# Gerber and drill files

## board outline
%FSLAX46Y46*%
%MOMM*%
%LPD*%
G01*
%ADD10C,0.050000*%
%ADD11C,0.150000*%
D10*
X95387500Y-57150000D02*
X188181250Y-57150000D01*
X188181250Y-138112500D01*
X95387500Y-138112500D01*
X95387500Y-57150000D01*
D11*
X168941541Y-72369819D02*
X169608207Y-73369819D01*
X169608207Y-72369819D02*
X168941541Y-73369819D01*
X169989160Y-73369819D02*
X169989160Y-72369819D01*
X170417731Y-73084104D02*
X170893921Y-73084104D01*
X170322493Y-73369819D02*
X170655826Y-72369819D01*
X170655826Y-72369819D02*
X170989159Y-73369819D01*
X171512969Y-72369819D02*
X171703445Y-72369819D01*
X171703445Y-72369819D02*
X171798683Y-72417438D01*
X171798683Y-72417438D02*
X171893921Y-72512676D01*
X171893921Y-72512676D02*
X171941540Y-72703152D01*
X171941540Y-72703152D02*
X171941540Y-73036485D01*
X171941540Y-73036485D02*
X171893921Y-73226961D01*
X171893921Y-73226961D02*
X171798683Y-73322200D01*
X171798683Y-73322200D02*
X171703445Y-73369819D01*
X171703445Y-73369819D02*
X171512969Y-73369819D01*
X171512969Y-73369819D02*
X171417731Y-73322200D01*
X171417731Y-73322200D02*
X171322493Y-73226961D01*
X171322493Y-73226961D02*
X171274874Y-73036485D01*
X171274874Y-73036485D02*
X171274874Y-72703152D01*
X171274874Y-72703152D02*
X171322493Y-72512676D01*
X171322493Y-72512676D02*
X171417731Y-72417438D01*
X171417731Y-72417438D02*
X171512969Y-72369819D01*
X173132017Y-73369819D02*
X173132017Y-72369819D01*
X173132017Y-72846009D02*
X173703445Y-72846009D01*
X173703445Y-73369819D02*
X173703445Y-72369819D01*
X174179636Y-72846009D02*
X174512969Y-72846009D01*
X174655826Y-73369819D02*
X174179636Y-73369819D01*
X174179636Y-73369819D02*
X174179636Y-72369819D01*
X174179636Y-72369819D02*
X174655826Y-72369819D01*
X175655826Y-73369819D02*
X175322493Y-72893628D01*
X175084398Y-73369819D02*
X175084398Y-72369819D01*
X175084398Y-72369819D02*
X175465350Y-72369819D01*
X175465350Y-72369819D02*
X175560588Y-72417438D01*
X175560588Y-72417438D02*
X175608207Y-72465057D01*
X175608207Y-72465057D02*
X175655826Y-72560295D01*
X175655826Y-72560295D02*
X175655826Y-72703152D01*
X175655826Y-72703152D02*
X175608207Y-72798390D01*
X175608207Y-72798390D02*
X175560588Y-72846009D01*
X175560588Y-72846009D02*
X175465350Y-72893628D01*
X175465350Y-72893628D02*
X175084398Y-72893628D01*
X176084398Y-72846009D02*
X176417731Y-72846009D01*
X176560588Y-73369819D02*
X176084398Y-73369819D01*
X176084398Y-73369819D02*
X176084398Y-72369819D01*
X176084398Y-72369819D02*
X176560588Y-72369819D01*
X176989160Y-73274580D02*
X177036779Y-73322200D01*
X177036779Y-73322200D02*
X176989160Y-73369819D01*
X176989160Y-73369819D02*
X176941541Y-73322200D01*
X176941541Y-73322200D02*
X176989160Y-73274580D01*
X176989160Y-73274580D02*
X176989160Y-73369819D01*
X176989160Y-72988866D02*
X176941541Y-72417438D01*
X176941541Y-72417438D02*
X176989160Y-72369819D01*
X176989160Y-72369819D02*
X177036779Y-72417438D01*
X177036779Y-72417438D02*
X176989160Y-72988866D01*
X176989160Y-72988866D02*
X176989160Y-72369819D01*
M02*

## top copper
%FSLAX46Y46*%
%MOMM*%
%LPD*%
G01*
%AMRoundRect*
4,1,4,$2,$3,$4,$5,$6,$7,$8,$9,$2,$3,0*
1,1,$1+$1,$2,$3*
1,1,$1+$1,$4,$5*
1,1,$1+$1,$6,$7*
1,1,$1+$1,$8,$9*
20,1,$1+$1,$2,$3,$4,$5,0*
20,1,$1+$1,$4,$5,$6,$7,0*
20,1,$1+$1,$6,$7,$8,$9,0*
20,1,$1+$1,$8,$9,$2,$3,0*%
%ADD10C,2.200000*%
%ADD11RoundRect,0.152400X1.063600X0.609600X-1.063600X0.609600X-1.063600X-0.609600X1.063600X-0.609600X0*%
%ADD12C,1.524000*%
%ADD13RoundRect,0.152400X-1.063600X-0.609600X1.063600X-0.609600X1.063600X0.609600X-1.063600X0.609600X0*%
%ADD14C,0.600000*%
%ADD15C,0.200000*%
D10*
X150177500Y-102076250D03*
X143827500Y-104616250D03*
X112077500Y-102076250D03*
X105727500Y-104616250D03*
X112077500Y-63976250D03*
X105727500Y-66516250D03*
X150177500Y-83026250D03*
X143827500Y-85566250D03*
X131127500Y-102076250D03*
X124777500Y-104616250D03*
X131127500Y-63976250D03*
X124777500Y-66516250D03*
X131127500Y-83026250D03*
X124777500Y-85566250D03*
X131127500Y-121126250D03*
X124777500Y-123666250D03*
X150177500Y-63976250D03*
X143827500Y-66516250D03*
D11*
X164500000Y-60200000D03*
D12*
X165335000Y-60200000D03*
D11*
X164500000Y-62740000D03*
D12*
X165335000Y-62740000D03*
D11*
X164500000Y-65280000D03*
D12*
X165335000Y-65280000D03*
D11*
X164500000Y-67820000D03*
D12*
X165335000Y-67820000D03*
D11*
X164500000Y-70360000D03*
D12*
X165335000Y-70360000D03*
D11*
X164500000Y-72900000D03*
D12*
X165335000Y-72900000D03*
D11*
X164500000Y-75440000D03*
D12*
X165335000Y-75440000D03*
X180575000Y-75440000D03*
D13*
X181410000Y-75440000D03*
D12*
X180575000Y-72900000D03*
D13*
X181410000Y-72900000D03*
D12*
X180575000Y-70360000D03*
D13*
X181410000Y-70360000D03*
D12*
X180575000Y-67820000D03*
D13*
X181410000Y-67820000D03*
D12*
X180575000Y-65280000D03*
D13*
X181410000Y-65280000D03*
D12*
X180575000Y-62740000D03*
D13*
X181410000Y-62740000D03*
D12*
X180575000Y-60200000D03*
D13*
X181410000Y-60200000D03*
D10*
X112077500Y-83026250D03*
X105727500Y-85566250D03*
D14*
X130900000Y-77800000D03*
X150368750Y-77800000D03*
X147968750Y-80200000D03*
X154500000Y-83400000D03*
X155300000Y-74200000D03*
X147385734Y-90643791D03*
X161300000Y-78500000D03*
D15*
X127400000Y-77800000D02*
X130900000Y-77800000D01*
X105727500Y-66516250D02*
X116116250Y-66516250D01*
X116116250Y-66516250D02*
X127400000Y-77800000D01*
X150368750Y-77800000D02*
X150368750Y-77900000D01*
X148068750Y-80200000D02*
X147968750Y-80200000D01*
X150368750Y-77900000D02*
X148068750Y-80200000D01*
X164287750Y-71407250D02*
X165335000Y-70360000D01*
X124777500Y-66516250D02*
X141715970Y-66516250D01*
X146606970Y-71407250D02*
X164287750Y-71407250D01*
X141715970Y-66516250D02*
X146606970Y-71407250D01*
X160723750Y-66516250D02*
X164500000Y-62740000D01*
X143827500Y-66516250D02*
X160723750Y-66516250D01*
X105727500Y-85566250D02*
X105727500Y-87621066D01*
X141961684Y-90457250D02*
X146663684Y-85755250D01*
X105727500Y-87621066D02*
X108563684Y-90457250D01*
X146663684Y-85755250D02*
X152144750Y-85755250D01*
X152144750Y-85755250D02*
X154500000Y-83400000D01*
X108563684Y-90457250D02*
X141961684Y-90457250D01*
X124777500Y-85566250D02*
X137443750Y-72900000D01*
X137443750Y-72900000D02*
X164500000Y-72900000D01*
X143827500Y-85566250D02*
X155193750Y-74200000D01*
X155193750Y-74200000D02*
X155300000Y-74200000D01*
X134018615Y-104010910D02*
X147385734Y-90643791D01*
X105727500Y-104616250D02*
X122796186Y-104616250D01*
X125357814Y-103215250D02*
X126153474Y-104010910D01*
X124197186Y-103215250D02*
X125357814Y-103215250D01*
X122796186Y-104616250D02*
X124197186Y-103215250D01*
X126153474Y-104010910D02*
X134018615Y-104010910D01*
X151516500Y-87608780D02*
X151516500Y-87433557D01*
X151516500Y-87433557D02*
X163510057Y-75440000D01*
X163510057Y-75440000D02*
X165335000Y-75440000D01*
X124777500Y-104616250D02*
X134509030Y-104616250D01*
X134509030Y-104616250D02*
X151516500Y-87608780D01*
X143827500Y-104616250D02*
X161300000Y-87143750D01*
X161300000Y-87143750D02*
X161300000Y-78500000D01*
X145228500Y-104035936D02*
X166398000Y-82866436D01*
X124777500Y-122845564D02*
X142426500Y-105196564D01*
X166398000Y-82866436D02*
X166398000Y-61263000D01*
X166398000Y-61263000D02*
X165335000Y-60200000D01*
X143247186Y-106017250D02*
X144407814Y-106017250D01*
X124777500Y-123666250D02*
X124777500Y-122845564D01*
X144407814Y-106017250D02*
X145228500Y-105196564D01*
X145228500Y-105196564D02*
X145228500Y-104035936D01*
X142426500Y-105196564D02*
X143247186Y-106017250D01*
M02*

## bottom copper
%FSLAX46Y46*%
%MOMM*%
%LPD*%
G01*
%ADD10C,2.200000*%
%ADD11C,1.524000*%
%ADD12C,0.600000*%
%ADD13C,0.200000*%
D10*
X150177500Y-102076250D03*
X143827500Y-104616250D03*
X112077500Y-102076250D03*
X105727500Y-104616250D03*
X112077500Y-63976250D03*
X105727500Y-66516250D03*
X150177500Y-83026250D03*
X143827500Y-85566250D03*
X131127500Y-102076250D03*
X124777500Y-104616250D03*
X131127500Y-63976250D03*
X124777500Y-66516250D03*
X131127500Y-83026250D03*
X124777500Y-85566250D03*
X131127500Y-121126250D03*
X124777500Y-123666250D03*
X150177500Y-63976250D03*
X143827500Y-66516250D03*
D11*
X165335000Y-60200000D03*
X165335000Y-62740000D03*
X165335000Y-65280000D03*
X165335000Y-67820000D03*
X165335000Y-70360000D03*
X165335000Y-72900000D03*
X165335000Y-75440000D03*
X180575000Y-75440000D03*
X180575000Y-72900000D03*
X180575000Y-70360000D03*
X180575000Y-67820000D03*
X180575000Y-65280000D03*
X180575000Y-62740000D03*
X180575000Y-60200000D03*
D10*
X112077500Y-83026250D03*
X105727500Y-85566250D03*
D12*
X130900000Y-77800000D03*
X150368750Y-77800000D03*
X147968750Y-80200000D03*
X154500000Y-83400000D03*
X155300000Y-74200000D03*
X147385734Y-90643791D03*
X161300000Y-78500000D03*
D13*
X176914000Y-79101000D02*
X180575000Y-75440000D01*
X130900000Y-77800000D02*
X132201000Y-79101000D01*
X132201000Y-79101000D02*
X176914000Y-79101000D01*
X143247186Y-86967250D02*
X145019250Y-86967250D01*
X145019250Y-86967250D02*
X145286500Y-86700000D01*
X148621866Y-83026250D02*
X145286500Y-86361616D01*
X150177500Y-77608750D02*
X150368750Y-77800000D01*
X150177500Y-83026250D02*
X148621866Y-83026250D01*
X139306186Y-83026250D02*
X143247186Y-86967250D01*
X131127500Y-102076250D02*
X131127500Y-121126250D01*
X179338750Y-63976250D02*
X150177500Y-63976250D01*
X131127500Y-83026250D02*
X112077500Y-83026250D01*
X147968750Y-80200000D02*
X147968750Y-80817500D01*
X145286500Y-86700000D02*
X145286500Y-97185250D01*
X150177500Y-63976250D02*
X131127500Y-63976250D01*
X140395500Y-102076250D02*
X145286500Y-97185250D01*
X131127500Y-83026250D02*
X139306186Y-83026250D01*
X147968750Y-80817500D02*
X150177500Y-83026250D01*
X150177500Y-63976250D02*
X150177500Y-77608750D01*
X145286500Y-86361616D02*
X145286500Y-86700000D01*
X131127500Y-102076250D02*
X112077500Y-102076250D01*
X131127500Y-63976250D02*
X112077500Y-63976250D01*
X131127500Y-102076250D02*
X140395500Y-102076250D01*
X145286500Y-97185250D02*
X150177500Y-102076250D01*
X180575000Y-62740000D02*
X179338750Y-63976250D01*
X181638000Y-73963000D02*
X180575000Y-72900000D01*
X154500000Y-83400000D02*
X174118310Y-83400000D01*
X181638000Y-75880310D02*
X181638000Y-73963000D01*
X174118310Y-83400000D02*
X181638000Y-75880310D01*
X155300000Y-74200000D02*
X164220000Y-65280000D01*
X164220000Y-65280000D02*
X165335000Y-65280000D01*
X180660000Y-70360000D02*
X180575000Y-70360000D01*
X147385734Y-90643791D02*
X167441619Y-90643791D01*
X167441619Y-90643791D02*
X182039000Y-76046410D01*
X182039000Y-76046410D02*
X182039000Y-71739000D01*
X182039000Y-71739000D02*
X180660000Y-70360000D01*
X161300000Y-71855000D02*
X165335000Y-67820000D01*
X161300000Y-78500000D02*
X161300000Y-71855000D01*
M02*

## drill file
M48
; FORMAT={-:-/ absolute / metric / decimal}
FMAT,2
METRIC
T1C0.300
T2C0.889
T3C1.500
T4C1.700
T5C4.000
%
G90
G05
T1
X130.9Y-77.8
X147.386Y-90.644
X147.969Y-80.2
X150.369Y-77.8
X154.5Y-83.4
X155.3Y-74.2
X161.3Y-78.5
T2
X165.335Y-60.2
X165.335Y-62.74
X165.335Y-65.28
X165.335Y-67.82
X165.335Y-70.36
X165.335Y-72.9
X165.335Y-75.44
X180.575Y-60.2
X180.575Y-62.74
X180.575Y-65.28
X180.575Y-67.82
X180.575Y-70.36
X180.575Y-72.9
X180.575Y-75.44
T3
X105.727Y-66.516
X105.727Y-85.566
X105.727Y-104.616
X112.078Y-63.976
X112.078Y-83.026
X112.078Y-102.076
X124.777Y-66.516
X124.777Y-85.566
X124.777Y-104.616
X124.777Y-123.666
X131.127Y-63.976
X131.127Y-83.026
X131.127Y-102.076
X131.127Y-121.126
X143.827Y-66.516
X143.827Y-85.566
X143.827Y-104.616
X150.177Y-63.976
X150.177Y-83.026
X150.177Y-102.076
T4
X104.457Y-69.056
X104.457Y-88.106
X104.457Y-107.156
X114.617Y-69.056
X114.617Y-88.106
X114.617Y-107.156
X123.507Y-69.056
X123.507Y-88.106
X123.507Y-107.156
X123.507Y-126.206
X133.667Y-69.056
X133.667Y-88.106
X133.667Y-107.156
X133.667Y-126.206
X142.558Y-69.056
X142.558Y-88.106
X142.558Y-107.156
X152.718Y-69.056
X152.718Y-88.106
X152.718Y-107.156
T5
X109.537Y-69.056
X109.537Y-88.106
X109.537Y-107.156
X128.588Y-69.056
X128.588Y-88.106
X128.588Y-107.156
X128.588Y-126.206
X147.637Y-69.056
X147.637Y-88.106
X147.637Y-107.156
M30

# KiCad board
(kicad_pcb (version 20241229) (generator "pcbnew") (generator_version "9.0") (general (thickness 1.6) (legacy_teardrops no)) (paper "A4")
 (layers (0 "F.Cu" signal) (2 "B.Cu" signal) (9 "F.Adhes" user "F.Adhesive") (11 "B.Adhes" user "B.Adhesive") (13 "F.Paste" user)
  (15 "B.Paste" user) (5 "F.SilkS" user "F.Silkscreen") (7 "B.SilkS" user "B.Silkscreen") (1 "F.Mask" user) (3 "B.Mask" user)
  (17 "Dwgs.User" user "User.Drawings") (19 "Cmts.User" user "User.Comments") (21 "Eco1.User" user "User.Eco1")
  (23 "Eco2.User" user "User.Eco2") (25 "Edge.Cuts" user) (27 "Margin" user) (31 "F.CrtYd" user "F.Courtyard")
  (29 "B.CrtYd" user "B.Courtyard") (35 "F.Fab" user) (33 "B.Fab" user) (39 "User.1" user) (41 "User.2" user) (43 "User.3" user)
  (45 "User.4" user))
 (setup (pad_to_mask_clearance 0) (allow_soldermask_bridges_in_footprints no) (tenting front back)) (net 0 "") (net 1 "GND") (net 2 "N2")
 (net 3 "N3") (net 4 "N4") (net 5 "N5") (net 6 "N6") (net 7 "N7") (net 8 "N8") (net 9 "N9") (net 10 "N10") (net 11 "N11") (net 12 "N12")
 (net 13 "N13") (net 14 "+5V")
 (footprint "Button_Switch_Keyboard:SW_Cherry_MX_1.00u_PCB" (layer "F.Cu") (at 150.1775 102.07625)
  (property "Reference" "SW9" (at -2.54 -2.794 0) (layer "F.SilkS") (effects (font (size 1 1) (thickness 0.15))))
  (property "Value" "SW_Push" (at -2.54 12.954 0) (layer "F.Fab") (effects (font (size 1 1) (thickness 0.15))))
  (pad "" np_thru_hole circle (at -7.62 5.08) (size 1.7 1.7) (drill 1.7) (layers "*.Cu" "*.Mask"))
  (pad "" np_thru_hole circle (at -2.54 5.08) (size 4 4) (drill 4) (layers "*.Cu" "*.Mask"))
  (pad "" np_thru_hole circle (at 2.54 5.08) (size 1.7 1.7) (drill 1.7) (layers "*.Cu" "*.Mask"))
  (pad "1" thru_hole circle (at 0 0) (size 2.2 2.2) (drill 1.5) (layers "*.Cu" "*.Mask") (remove_unused_layers no) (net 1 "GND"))
  (pad "2" thru_hole circle (at -6.35 2.54) (size 2.2 2.2) (drill 1.5) (layers "*.Cu" "*.Mask") (remove_unused_layers no) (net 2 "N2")))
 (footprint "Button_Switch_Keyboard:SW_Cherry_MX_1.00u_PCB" (layer "F.Cu") (at 112.0775 102.07625)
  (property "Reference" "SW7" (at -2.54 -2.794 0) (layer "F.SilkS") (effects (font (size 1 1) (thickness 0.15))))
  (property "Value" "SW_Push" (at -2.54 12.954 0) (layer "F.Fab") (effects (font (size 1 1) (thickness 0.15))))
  (pad "" np_thru_hole circle (at -7.62 5.08) (size 1.7 1.7) (drill 1.7) (layers "*.Cu" "*.Mask"))
  (pad "" np_thru_hole circle (at -2.54 5.08) (size 4 4) (drill 4) (layers "*.Cu" "*.Mask"))
  (pad "" np_thru_hole circle (at 2.54 5.08) (size 1.7 1.7) (drill 1.7) (layers "*.Cu" "*.Mask"))
  (pad "1" thru_hole circle (at 0 0) (size 2.2 2.2) (drill 1.5) (layers "*.Cu" "*.Mask") (remove_unused_layers no) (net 1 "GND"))
  (pad "2" thru_hole circle (at -6.35 2.54) (size 2.2 2.2) (drill 1.5) (layers "*.Cu" "*.Mask") (remove_unused_layers no) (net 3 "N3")))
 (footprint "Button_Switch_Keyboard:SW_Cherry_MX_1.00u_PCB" (layer "F.Cu") (at 112.0775 63.97625)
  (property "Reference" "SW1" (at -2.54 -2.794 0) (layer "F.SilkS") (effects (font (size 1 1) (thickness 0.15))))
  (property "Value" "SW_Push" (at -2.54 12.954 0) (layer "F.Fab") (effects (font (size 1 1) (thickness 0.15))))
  (pad "" np_thru_hole circle (at -7.62 5.08) (size 1.7 1.7) (drill 1.7) (layers "*.Cu" "*.Mask"))
  (pad "" np_thru_hole circle (at -2.54 5.08) (size 4 4) (drill 4) (layers "*.Cu" "*.Mask"))
  (pad "" np_thru_hole circle (at 2.54 5.08) (size 1.7 1.7) (drill 1.7) (layers "*.Cu" "*.Mask"))
  (pad "1" thru_hole circle (at 0 0) (size 2.2 2.2) (drill 1.5) (layers "*.Cu" "*.Mask") (remove_unused_layers no) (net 1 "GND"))
  (pad "2" thru_hole circle (at -6.35 2.54) (size 2.2 2.2) (drill 1.5) (layers "*.Cu" "*.Mask") (remove_unused_layers no) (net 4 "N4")))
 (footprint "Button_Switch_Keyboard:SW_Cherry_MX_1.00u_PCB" (layer "F.Cu") (at 150.1775 83.02625)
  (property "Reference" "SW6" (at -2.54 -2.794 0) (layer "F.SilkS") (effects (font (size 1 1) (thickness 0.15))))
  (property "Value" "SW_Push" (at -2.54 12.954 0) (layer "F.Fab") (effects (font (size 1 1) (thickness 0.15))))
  (pad "" np_thru_hole circle (at -7.62 5.08) (size 1.7 1.7) (drill 1.7) (layers "*.Cu" "*.Mask"))
  (pad "" np_thru_hole circle (at -2.54 5.08) (size 4 4) (drill 4) (layers "*.Cu" "*.Mask"))
  (pad "" np_thru_hole circle (at 2.54 5.08) (size 1.7 1.7) (drill 1.7) (layers "*.Cu" "*.Mask"))
  (pad "1" thru_hole circle (at 0 0) (size 2.2 2.2) (drill 1.5) (layers "*.Cu" "*.Mask") (remove_unused_layers no) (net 1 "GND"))
  (pad "2" thru_hole circle (at -6.35 2.54) (size 2.2 2.2) (drill 1.5) (layers "*.Cu" "*.Mask") (remove_unused_layers no) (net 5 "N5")))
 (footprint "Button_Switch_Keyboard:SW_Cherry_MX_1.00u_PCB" (layer "F.Cu") (at 131.1275 102.07625)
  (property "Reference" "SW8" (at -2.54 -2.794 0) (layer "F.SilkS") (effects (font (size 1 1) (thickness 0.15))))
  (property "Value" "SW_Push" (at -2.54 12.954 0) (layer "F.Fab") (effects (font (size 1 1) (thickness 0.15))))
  (pad "" np_thru_hole circle (at -7.62 5.08) (size 1.7 1.7) (drill 1.7) (layers "*.Cu" "*.Mask"))
  (pad "" np_thru_hole circle (at -2.54 5.08) (size 4 4) (drill 4) (layers "*.Cu" "*.Mask"))
  (pad "" np_thru_hole circle (at 2.54 5.08) (size 1.7 1.7) (drill 1.7) (layers "*.Cu" "*.Mask"))
  (pad "1" thru_hole circle (at 0 0) (size 2.2 2.2) (drill 1.5) (layers "*.Cu" "*.Mask") (remove_unused_layers no) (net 1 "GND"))
  (pad "2" thru_hole circle (at -6.35 2.54) (size 2.2 2.2) (drill 1.5) (layers "*.Cu" "*.Mask") (remove_unused_layers no) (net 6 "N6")))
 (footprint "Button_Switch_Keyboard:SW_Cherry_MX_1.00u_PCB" (layer "F.Cu") (at 131.1275 63.97625)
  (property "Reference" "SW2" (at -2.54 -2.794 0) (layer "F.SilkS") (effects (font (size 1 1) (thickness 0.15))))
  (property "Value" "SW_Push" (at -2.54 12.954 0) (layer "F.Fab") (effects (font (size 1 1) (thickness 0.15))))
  (pad "" np_thru_hole circle (at -7.62 5.08) (size 1.7 1.7) (drill 1.7) (layers "*.Cu" "*.Mask"))
  (pad "" np_thru_hole circle (at -2.54 5.08) (size 4 4) (drill 4) (layers "*.Cu" "*.Mask"))
  (pad "" np_thru_hole circle (at 2.54 5.08) (size 1.7 1.7) (drill 1.7) (layers "*.Cu" "*.Mask"))
  (pad "1" thru_hole circle (at 0 0) (size 2.2 2.2) (drill 1.5) (layers "*.Cu" "*.Mask") (remove_unused_layers no) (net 1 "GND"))
  (pad "2" thru_hole circle (at -6.35 2.54) (size 2.2 2.2) (drill 1.5) (layers "*.Cu" "*.Mask") (remove_unused_layers no) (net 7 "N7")))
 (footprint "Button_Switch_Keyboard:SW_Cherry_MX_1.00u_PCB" (layer "F.Cu") (at 131.1275 83.02625)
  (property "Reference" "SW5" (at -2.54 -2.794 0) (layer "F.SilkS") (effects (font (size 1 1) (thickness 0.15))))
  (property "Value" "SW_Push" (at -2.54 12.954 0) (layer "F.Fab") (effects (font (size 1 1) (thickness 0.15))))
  (pad "" np_thru_hole circle (at -7.62 5.08) (size 1.7 1.7) (drill 1.7) (layers "*.Cu" "*.Mask"))
  (pad "" np_thru_hole circle (at -2.54 5.08) (size 4 4) (drill 4) (layers "*.Cu" "*.Mask"))
  (pad "" np_thru_hole circle (at 2.54 5.08) (size 1.7 1.7) (drill 1.7) (layers "*.Cu" "*.Mask"))
  (pad "1" thru_hole circle (at 0 0) (size 2.2 2.2) (drill 1.5) (layers "*.Cu" "*.Mask") (remove_unused_layers no) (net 1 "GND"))
  (pad "2" thru_hole circle (at -6.35 2.54) (size 2.2 2.2) (drill 1.5) (layers "*.Cu" "*.Mask") (remove_unused_layers no) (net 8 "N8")))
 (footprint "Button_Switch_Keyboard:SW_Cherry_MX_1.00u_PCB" (layer "F.Cu") (at 131.1275 121.12625)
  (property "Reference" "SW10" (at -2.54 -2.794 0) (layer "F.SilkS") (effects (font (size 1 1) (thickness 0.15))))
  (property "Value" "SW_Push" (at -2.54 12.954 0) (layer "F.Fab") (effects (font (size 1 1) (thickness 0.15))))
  (pad "" np_thru_hole circle (at -7.62 5.08) (size 1.7 1.7) (drill 1.7) (layers "*.Cu" "*.Mask"))
  (pad "" np_thru_hole circle (at -2.54 5.08) (size 4 4) (drill 4) (layers "*.Cu" "*.Mask"))
  (pad "" np_thru_hole circle (at 2.54 5.08) (size 1.7 1.7) (drill 1.7) (layers "*.Cu" "*.Mask"))
  (pad "1" thru_hole circle (at 0 0) (size 2.2 2.2) (drill 1.5) (layers "*.Cu" "*.Mask") (remove_unused_layers no) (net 1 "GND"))
  (pad "2" thru_hole circle (at -6.35 2.54) (size 2.2 2.2) (drill 1.5) (layers "*.Cu" "*.Mask") (remove_unused_layers no) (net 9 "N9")))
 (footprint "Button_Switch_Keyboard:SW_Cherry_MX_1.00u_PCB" (layer "F.Cu") (at 150.1775 63.97625)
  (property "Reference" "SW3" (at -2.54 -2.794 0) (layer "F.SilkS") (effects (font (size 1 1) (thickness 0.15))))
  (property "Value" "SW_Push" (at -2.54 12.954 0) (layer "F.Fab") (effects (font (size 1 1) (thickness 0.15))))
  (pad "" np_thru_hole circle (at -7.62 5.08) (size 1.7 1.7) (drill 1.7) (layers "*.Cu" "*.Mask"))
  (pad "" np_thru_hole circle (at -2.54 5.08) (size 4 4) (drill 4) (layers "*.Cu" "*.Mask"))
  (pad "" np_thru_hole circle (at 2.54 5.08) (size 1.7 1.7) (drill 1.7) (layers "*.Cu" "*.Mask"))
  (pad "1" thru_hole circle (at 0 0) (size 2.2 2.2) (drill 1.5) (layers "*.Cu" "*.Mask") (remove_unused_layers no) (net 1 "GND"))
  (pad "2" thru_hole circle (at -6.35 2.54) (size 2.2 2.2) (drill 1.5) (layers "*.Cu" "*.Mask") (remove_unused_layers no) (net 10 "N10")))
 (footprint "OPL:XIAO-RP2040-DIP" (layer "F.Cu") (at 172.955 67.82)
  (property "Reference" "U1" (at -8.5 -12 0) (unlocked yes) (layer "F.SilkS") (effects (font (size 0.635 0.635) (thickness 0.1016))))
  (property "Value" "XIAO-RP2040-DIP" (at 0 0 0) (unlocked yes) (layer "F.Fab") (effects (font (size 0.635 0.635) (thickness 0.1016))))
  (pad "1" smd roundrect (at -8.455 -7.62 180) (size 2.432 1.524) (layers "F.Cu" "F.Mask") (roundrect_rratio 0.1) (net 9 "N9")
   (thermal_bridge_angle 45))
  (pad "1" thru_hole circle (at -7.62 -7.62 180) (size 1.524 1.524) (drill 0.889) (layers "*.Cu" "*.Mask") (remove_unused_layers no)
   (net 9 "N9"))
  (pad "2" smd roundrect (at -8.455 -5.08 180) (size 2.432 1.524) (layers "F.Cu" "F.Mask") (roundrect_rratio 0.1) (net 10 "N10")
   (thermal_bridge_angle 45))
  (pad "2" thru_hole circle (at -7.62 -5.08 180) (size 1.524 1.524) (drill 0.889) (layers "*.Cu" "*.Mask") (remove_unused_layers no)
   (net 10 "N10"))
  (pad "3" smd roundrect (at -8.455 -2.54 180) (size 2.432 1.524) (layers "F.Cu" "F.Mask") (roundrect_rratio 0.1) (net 5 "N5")
   (thermal_bridge_angle 45))
  (pad "3" thru_hole circle (at -7.62 -2.54 180) (size 1.524 1.524) (drill 0.889) (layers "*.Cu" "*.Mask") (remove_unused_layers no)
   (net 5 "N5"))
  (pad "4" smd roundrect (at -8.455 0 180) (size 2.432 1.524) (layers "F.Cu" "F.Mask") (roundrect_rratio 0.1) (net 2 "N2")
   (thermal_bridge_angle 45))
  (pad "4" thru_hole circle (at -7.62 0 180) (size 1.524 1.524) (drill 0.889) (layers "*.Cu" "*.Mask") (remove_unused_layers no)
   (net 2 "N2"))
  (pad "5" smd roundrect (at -8.455 2.54 180) (size 2.432 1.524) (layers "F.Cu" "F.Mask") (roundrect_rratio 0.1) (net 7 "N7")
   (thermal_bridge_angle 45))
  (pad "5" thru_hole circle (at -7.62 2.54 180) (size 1.524 1.524) (drill 0.889) (layers "*.Cu" "*.Mask") (remove_unused_layers no)
   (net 7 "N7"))
  (pad "6" smd roundrect (at -8.455 5.08 180) (size 2.432 1.524) (layers "F.Cu" "F.Mask") (roundrect_rratio 0.1) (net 8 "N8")
   (thermal_bridge_angle 45))
  (pad "6" thru_hole circle (at -7.62 5.08 180) (size 1.524 1.524) (drill 0.889) (layers "*.Cu" "*.Mask") (remove_unused_layers no)
   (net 8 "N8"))
  (pad "7" smd roundrect (at -8.455 7.62 180) (size 2.432 1.524) (layers "F.Cu" "F.Mask") (roundrect_rratio 0.1) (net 6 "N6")
   (thermal_bridge_angle 45))
  (pad "7" thru_hole circle (at -7.62 7.62 180) (size 1.524 1.524) (drill 0.889) (layers "*.Cu" "*.Mask") (remove_unused_layers no)
   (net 6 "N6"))
  (pad "8" thru_hole circle (at 7.62 7.62) (size 1.524 1.524) (drill 0.889) (layers "*.Cu" "*.Mask") (remove_unused_layers no) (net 4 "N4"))
  (pad "8" smd roundrect (at 8.455 7.62) (size 2.432 1.524) (layers "F.Cu" "F.Mask") (roundrect_rratio 0.1) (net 4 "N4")
   (thermal_bridge_angle 45))
  (pad "9" thru_hole circle (at 7.62 5.08) (size 1.524 1.524) (drill 0.889) (layers "*.Cu" "*.Mask") (remove_unused_layers no)
   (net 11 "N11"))
  (pad "9" smd roundrect (at 8.455 5.08) (size 2.432 1.524) (layers "F.Cu" "F.Mask") (roundrect_rratio 0.1) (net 11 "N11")
   (thermal_bridge_angle 45))
  (pad "10" thru_hole circle (at 7.62 2.54) (size 1.524 1.524) (drill 0.889) (layers "*.Cu" "*.Mask") (remove_unused_layers no) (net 3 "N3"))
  (pad "10" smd roundrect (at 8.455 2.54) (size 2.432 1.524) (layers "F.Cu" "F.Mask") (roundrect_rratio 0.1) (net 3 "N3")
   (thermal_bridge_angle 45))
  (pad "11" thru_hole circle (at 7.62 0) (size 1.524 1.524) (drill 0.889) (layers "*.Cu" "*.Mask") (remove_unused_layers no) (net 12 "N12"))
  (pad "11" smd roundrect (at 8.455 0) (size 2.432 1.524) (layers "F.Cu" "F.Mask") (roundrect_rratio 0.1) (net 12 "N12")
   (thermal_bridge_angle 45))
  (pad "12" thru_hole circle (at 7.62 -2.54) (size 1.524 1.524) (drill 0.889) (layers "*.Cu" "*.Mask") (remove_unused_layers no)
   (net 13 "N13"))
  (pad "12" smd roundrect (at 8.455 -2.54) (size 2.432 1.524) (layers "F.Cu" "F.Mask") (roundrect_rratio 0.1) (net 13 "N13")
   (thermal_bridge_angle 45))
  (pad "13" thru_hole circle (at 7.62 -5.08) (size 1.524 1.524) (drill 0.889) (layers "*.Cu" "*.Mask") (remove_unused_layers no)
   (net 1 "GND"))
  (pad "13" smd roundrect (at 8.455 -5.08) (size 2.432 1.524) (layers "F.Cu" "F.Mask") (roundrect_rratio 0.1) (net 1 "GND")
   (thermal_bridge_angle 45))
  (pad "14" thru_hole circle (at 7.62 -7.62) (size 1.524 1.524) (drill 0.889) (layers "*.Cu" "*.Mask") (remove_unused_layers no)
   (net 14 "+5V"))
  (pad "14" smd roundrect (at 8.455 -7.62) (size 2.432 1.524) (layers "F.Cu" "F.Mask") (roundrect_rratio 0.1) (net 14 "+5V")
   (thermal_bridge_angle 45)))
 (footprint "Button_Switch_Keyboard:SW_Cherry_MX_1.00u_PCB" (layer "F.Cu") (at 112.0775 83.02625)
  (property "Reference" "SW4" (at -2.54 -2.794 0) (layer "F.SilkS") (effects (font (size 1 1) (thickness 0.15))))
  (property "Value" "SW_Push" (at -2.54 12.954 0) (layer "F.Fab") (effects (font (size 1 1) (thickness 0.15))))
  (pad "" np_thru_hole circle (at -7.62 5.08) (size 1.7 1.7) (drill 1.7) (layers "*.Cu" "*.Mask"))
  (pad "" np_thru_hole circle (at -2.54 5.08) (size 4 4) (drill 4) (layers "*.Cu" "*.Mask"))
  (pad "" np_thru_hole circle (at 2.54 5.08) (size 1.7 1.7) (drill 1.7) (layers "*.Cu" "*.Mask"))
  (pad "1" thru_hole circle (at 0 0) (size 2.2 2.2) (drill 1.5) (layers "*.Cu" "*.Mask") (remove_unused_layers no) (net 1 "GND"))
  (pad "2" thru_hole circle (at -6.35 2.54) (size 2.2 2.2) (drill 1.5) (layers "*.Cu" "*.Mask") (remove_unused_layers no) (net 11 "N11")))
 (gr_rect (start 95.3875 57.15) (end 188.18125 138.1125) (stroke (width 0.05) (type solid)) (fill no) (layer "Edge.Cuts"))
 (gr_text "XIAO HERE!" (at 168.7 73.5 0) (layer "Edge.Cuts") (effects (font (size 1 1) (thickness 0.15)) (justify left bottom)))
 (segment (start 127.4 77.8) (end 130.9 77.8) (width 0.2) (layer "F.Cu") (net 4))
 (segment (start 105.7275 66.51625) (end 116.11625 66.51625) (width 0.2) (layer "F.Cu") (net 4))
 (segment (start 116.11625 66.51625) (end 127.4 77.8) (width 0.2) (layer "F.Cu") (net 4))
 (via (at 130.9 77.8) (size 0.6) (drill 0.3) (layers "F.Cu" "B.Cu") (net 4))
 (segment (start 176.914 79.101) (end 180.575 75.44) (width 0.2) (layer "B.Cu") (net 4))
 (segment (start 130.9 77.8) (end 132.201 79.101) (width 0.2) (layer "B.Cu") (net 4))
 (segment (start 132.201 79.101) (end 176.914 79.101) (width 0.2) (layer "B.Cu") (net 4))
 (segment (start 150.36875 77.8) (end 150.36875 77.9) (width 0.2) (layer "F.Cu") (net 1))
 (segment (start 148.06875 80.2) (end 147.96875 80.2) (width 0.2) (layer "F.Cu") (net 1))
 (segment (start 150.36875 77.9) (end 148.06875 80.2) (width 0.2) (layer "F.Cu") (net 1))
 (via (at 150.36875 77.8) (size 0.6) (drill 0.3) (layers "F.Cu" "B.Cu") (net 1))
 (via (at 147.96875 80.2) (size 0.6) (drill 0.3) (layers "F.Cu" "B.Cu") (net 1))
 (segment (start 143.247186 86.96725) (end 145.01925 86.96725) (width 0.2) (layer "B.Cu") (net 1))
 (segment (start 145.01925 86.96725) (end 145.2865 86.7) (width 0.2) (layer "B.Cu") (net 1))
 (segment (start 148.621866 83.02625) (end 145.2865 86.361616) (width 0.2) (layer "B.Cu") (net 1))
 (segment (start 150.1775 77.60875) (end 150.36875 77.8) (width 0.2) (layer "B.Cu") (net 1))
 (segment (start 150.1775 83.02625) (end 148.621866 83.02625) (width 0.2) (layer "B.Cu") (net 1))
 (segment (start 139.306186 83.02625) (end 143.247186 86.96725) (width 0.2) (layer "B.Cu") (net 1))
 (segment (start 131.1275 102.07625) (end 131.1275 121.12625) (width 0.2) (layer "B.Cu") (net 1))
 (segment (start 179.33875 63.97625) (end 150.1775 63.97625) (width 0.2) (layer "B.Cu") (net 1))
 (segment (start 131.1275 83.02625) (end 112.0775 83.02625) (width 0.2) (layer "B.Cu") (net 1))
 (segment (start 147.96875 80.2) (end 147.96875 80.8175) (width 0.2) (layer "B.Cu") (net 1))
 (segment (start 145.2865 86.7) (end 145.2865 97.18525) (width 0.2) (layer "B.Cu") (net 1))
 (segment (start 150.1775 63.97625) (end 131.1275 63.97625) (width 0.2) (layer "B.Cu") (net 1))
 (segment (start 140.3955 102.07625) (end 145.2865 97.18525) (width 0.2) (layer "B.Cu") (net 1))
 (segment (start 131.1275 83.02625) (end 139.306186 83.02625) (width 0.2) (layer "B.Cu") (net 1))
 (segment (start 147.96875 80.8175) (end 150.1775 83.02625) (width 0.2) (layer "B.Cu") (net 1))
 (segment (start 150.1775 63.97625) (end 150.1775 77.60875) (width 0.2) (layer "B.Cu") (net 1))
 (segment (start 145.2865 86.361616) (end 145.2865 86.7) (width 0.2) (layer "B.Cu") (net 1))
 (segment (start 131.1275 102.07625) (end 112.0775 102.07625) (width 0.2) (layer "B.Cu") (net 1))
 (segment (start 131.1275 63.97625) (end 112.0775 63.97625) (width 0.2) (layer "B.Cu") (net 1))
 (segment (start 131.1275 102.07625) (end 140.3955 102.07625) (width 0.2) (layer "B.Cu") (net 1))
 (segment (start 145.2865 97.18525) (end 150.1775 102.07625) (width 0.2) (layer "B.Cu") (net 1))
 (segment (start 180.575 62.74) (end 179.33875 63.97625) (width 0.2) (layer "B.Cu") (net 1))
 (segment (start 164.28775 71.40725) (end 165.335 70.36) (width 0.2) (layer "F.Cu") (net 7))
 (segment (start 124.7775 66.51625) (end 141.71597 66.51625) (width 0.2) (layer "F.Cu") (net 7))
 (segment (start 146.60697 71.40725) (end 164.28775 71.40725) (width 0.2) (layer "F.Cu") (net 7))
 (segment (start 141.71597 66.51625) (end 146.60697 71.40725) (width 0.2) (layer "F.Cu") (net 7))
 (segment (start 160.72375 66.51625) (end 164.5 62.74) (width 0.2) (layer "F.Cu") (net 10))
 (segment (start 143.8275 66.51625) (end 160.72375 66.51625) (width 0.2) (layer "F.Cu") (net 10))
 (segment (start 105.7275 85.56625) (end 105.7275 87.621066) (width 0.2) (layer "F.Cu") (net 11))
 (segment (start 141.961684 90.45725) (end 146.663684 85.75525) (width 0.2) (layer "F.Cu") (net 11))
 (segment (start 105.7275 87.621066) (end 108.563684 90.45725) (width 0.2) (layer "F.Cu") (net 11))
 (segment (start 146.663684 85.75525) (end 152.14475 85.75525) (width 0.2) (layer "F.Cu") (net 11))
 (segment (start 152.14475 85.75525) (end 154.5 83.4) (width 0.2) (layer "F.Cu") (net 11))
 (segment (start 108.563684 90.45725) (end 141.961684 90.45725) (width 0.2) (layer "F.Cu") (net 11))
 (via (at 154.5 83.4) (size 0.6) (drill 0.3) (layers "F.Cu" "B.Cu") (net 11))
 (segment (start 181.638 73.963) (end 180.575 72.9) (width 0.2) (layer "B.Cu") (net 11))
 (segment (start 154.5 83.4) (end 174.11831 83.4) (width 0.2) (layer "B.Cu") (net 11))
 (segment (start 181.638 75.88031) (end 181.638 73.963) (width 0.2) (layer "B.Cu") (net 11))
 (segment (start 174.11831 83.4) (end 181.638 75.88031) (width 0.2) (layer "B.Cu") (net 11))
 (segment (start 124.7775 85.56625) (end 137.44375 72.9) (width 0.2) (layer "F.Cu") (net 8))
 (segment (start 137.44375 72.9) (end 164.5 72.9) (width 0.2) (layer "F.Cu") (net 8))
 (segment (start 143.8275 85.56625) (end 155.19375 74.2) (width 0.2) (layer "F.Cu") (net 5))
 (segment (start 155.19375 74.2) (end 155.3 74.2) (width 0.2) (layer "F.Cu") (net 5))
 (via (at 155.3 74.2) (size 0.6) (drill 0.3) (layers "F.Cu" "B.Cu") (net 5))
 (segment (start 155.3 74.2) (end 164.22 65.28) (width 0.2) (layer "B.Cu") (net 5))
 (segment (start 164.22 65.28) (end 165.335 65.28) (width 0.2) (layer "B.Cu") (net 5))
 (segment (start 134.018615 104.01091) (end 147.385734 90.643791) (width 0.2) (layer "F.Cu") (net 3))
 (segment (start 105.7275 104.61625) (end 122.796186 104.61625) (width 0.2) (layer "F.Cu") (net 3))
 (segment (start 125.357814 103.21525) (end 126.153474 104.01091) (width 0.2) (layer "F.Cu") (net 3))
 (segment (start 124.197186 103.21525) (end 125.357814 103.21525) (width 0.2) (layer "F.Cu") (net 3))
 (segment (start 122.796186 104.61625) (end 124.197186 103.21525) (width 0.2) (layer "F.Cu") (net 3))
 (segment (start 126.153474 104.01091) (end 134.018615 104.01091) (width 0.2) (layer "F.Cu") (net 3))
 (via (at 147.385734 90.643791) (size 0.6) (drill 0.3) (layers "F.Cu" "B.Cu") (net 3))
 (segment (start 180.66 70.36) (end 180.575 70.36) (width 0.2) (layer "B.Cu") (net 3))
 (segment (start 147.385734 90.643791) (end 167.441619 90.643791) (width 0.2) (layer "B.Cu") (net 3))
 (segment (start 167.441619 90.643791) (end 182.039 76.04641) (width 0.2) (layer "B.Cu") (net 3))
 (segment (start 182.039 76.04641) (end 182.039 71.739) (width 0.2) (layer "B.Cu") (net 3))
 (segment (start 182.039 71.739) (end 180.66 70.36) (width 0.2) (layer "B.Cu") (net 3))
 (segment (start 151.5165 87.60878) (end 151.5165 87.433557) (width 0.2) (layer "F.Cu") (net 6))
 (segment (start 151.5165 87.433557) (end 163.510057 75.44) (width 0.2) (layer "F.Cu") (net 6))
 (segment (start 163.510057 75.44) (end 165.335 75.44) (width 0.2) (layer "F.Cu") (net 6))
 (segment (start 124.7775 104.61625) (end 134.50903 104.61625) (width 0.2) (layer "F.Cu") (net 6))
 (segment (start 134.50903 104.61625) (end 151.5165 87.60878) (width 0.2) (layer "F.Cu") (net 6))
 (segment (start 143.8275 104.61625) (end 161.3 87.14375) (width 0.2) (layer "F.Cu") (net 2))
 (segment (start 161.3 87.14375) (end 161.3 78.5) (width 0.2) (layer "F.Cu") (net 2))
 (via (at 161.3 78.5) (size 0.6) (drill 0.3) (layers "F.Cu" "B.Cu") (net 2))
 (segment (start 161.3 71.855) (end 165.335 67.82) (width 0.2) (layer "B.Cu") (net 2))
 (segment (start 161.3 78.5) (end 161.3 71.855) (width 0.2) (layer "B.Cu") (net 2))
 (segment (start 145.2285 104.035936) (end 166.398 82.866436) (width 0.2) (layer "F.Cu") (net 9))
 (segment (start 124.7775 122.845564) (end 142.4265 105.196564) (width 0.2) (layer "F.Cu") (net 9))
 (segment (start 166.398 82.866436) (end 166.398 61.263) (width 0.2) (layer "F.Cu") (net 9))
 (segment (start 166.398 61.263) (end 165.335 60.2) (width 0.2) (layer "F.Cu") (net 9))
 (segment (start 143.247186 106.01725) (end 144.407814 106.01725) (width 0.2) (layer "F.Cu") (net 9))
 (segment (start 124.7775 123.66625) (end 124.7775 122.845564) (width 0.2) (layer "F.Cu") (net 9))
 (segment (start 144.407814 106.01725) (end 145.2285 105.196564) (width 0.2) (layer "F.Cu") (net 9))
 (segment (start 145.2285 105.196564) (end 145.2285 104.035936) (width 0.2) (layer "F.Cu") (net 9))
 (segment (start 142.4265 105.196564) (end 143.247186 106.01725) (width 0.2) (layer "F.Cu") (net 9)))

